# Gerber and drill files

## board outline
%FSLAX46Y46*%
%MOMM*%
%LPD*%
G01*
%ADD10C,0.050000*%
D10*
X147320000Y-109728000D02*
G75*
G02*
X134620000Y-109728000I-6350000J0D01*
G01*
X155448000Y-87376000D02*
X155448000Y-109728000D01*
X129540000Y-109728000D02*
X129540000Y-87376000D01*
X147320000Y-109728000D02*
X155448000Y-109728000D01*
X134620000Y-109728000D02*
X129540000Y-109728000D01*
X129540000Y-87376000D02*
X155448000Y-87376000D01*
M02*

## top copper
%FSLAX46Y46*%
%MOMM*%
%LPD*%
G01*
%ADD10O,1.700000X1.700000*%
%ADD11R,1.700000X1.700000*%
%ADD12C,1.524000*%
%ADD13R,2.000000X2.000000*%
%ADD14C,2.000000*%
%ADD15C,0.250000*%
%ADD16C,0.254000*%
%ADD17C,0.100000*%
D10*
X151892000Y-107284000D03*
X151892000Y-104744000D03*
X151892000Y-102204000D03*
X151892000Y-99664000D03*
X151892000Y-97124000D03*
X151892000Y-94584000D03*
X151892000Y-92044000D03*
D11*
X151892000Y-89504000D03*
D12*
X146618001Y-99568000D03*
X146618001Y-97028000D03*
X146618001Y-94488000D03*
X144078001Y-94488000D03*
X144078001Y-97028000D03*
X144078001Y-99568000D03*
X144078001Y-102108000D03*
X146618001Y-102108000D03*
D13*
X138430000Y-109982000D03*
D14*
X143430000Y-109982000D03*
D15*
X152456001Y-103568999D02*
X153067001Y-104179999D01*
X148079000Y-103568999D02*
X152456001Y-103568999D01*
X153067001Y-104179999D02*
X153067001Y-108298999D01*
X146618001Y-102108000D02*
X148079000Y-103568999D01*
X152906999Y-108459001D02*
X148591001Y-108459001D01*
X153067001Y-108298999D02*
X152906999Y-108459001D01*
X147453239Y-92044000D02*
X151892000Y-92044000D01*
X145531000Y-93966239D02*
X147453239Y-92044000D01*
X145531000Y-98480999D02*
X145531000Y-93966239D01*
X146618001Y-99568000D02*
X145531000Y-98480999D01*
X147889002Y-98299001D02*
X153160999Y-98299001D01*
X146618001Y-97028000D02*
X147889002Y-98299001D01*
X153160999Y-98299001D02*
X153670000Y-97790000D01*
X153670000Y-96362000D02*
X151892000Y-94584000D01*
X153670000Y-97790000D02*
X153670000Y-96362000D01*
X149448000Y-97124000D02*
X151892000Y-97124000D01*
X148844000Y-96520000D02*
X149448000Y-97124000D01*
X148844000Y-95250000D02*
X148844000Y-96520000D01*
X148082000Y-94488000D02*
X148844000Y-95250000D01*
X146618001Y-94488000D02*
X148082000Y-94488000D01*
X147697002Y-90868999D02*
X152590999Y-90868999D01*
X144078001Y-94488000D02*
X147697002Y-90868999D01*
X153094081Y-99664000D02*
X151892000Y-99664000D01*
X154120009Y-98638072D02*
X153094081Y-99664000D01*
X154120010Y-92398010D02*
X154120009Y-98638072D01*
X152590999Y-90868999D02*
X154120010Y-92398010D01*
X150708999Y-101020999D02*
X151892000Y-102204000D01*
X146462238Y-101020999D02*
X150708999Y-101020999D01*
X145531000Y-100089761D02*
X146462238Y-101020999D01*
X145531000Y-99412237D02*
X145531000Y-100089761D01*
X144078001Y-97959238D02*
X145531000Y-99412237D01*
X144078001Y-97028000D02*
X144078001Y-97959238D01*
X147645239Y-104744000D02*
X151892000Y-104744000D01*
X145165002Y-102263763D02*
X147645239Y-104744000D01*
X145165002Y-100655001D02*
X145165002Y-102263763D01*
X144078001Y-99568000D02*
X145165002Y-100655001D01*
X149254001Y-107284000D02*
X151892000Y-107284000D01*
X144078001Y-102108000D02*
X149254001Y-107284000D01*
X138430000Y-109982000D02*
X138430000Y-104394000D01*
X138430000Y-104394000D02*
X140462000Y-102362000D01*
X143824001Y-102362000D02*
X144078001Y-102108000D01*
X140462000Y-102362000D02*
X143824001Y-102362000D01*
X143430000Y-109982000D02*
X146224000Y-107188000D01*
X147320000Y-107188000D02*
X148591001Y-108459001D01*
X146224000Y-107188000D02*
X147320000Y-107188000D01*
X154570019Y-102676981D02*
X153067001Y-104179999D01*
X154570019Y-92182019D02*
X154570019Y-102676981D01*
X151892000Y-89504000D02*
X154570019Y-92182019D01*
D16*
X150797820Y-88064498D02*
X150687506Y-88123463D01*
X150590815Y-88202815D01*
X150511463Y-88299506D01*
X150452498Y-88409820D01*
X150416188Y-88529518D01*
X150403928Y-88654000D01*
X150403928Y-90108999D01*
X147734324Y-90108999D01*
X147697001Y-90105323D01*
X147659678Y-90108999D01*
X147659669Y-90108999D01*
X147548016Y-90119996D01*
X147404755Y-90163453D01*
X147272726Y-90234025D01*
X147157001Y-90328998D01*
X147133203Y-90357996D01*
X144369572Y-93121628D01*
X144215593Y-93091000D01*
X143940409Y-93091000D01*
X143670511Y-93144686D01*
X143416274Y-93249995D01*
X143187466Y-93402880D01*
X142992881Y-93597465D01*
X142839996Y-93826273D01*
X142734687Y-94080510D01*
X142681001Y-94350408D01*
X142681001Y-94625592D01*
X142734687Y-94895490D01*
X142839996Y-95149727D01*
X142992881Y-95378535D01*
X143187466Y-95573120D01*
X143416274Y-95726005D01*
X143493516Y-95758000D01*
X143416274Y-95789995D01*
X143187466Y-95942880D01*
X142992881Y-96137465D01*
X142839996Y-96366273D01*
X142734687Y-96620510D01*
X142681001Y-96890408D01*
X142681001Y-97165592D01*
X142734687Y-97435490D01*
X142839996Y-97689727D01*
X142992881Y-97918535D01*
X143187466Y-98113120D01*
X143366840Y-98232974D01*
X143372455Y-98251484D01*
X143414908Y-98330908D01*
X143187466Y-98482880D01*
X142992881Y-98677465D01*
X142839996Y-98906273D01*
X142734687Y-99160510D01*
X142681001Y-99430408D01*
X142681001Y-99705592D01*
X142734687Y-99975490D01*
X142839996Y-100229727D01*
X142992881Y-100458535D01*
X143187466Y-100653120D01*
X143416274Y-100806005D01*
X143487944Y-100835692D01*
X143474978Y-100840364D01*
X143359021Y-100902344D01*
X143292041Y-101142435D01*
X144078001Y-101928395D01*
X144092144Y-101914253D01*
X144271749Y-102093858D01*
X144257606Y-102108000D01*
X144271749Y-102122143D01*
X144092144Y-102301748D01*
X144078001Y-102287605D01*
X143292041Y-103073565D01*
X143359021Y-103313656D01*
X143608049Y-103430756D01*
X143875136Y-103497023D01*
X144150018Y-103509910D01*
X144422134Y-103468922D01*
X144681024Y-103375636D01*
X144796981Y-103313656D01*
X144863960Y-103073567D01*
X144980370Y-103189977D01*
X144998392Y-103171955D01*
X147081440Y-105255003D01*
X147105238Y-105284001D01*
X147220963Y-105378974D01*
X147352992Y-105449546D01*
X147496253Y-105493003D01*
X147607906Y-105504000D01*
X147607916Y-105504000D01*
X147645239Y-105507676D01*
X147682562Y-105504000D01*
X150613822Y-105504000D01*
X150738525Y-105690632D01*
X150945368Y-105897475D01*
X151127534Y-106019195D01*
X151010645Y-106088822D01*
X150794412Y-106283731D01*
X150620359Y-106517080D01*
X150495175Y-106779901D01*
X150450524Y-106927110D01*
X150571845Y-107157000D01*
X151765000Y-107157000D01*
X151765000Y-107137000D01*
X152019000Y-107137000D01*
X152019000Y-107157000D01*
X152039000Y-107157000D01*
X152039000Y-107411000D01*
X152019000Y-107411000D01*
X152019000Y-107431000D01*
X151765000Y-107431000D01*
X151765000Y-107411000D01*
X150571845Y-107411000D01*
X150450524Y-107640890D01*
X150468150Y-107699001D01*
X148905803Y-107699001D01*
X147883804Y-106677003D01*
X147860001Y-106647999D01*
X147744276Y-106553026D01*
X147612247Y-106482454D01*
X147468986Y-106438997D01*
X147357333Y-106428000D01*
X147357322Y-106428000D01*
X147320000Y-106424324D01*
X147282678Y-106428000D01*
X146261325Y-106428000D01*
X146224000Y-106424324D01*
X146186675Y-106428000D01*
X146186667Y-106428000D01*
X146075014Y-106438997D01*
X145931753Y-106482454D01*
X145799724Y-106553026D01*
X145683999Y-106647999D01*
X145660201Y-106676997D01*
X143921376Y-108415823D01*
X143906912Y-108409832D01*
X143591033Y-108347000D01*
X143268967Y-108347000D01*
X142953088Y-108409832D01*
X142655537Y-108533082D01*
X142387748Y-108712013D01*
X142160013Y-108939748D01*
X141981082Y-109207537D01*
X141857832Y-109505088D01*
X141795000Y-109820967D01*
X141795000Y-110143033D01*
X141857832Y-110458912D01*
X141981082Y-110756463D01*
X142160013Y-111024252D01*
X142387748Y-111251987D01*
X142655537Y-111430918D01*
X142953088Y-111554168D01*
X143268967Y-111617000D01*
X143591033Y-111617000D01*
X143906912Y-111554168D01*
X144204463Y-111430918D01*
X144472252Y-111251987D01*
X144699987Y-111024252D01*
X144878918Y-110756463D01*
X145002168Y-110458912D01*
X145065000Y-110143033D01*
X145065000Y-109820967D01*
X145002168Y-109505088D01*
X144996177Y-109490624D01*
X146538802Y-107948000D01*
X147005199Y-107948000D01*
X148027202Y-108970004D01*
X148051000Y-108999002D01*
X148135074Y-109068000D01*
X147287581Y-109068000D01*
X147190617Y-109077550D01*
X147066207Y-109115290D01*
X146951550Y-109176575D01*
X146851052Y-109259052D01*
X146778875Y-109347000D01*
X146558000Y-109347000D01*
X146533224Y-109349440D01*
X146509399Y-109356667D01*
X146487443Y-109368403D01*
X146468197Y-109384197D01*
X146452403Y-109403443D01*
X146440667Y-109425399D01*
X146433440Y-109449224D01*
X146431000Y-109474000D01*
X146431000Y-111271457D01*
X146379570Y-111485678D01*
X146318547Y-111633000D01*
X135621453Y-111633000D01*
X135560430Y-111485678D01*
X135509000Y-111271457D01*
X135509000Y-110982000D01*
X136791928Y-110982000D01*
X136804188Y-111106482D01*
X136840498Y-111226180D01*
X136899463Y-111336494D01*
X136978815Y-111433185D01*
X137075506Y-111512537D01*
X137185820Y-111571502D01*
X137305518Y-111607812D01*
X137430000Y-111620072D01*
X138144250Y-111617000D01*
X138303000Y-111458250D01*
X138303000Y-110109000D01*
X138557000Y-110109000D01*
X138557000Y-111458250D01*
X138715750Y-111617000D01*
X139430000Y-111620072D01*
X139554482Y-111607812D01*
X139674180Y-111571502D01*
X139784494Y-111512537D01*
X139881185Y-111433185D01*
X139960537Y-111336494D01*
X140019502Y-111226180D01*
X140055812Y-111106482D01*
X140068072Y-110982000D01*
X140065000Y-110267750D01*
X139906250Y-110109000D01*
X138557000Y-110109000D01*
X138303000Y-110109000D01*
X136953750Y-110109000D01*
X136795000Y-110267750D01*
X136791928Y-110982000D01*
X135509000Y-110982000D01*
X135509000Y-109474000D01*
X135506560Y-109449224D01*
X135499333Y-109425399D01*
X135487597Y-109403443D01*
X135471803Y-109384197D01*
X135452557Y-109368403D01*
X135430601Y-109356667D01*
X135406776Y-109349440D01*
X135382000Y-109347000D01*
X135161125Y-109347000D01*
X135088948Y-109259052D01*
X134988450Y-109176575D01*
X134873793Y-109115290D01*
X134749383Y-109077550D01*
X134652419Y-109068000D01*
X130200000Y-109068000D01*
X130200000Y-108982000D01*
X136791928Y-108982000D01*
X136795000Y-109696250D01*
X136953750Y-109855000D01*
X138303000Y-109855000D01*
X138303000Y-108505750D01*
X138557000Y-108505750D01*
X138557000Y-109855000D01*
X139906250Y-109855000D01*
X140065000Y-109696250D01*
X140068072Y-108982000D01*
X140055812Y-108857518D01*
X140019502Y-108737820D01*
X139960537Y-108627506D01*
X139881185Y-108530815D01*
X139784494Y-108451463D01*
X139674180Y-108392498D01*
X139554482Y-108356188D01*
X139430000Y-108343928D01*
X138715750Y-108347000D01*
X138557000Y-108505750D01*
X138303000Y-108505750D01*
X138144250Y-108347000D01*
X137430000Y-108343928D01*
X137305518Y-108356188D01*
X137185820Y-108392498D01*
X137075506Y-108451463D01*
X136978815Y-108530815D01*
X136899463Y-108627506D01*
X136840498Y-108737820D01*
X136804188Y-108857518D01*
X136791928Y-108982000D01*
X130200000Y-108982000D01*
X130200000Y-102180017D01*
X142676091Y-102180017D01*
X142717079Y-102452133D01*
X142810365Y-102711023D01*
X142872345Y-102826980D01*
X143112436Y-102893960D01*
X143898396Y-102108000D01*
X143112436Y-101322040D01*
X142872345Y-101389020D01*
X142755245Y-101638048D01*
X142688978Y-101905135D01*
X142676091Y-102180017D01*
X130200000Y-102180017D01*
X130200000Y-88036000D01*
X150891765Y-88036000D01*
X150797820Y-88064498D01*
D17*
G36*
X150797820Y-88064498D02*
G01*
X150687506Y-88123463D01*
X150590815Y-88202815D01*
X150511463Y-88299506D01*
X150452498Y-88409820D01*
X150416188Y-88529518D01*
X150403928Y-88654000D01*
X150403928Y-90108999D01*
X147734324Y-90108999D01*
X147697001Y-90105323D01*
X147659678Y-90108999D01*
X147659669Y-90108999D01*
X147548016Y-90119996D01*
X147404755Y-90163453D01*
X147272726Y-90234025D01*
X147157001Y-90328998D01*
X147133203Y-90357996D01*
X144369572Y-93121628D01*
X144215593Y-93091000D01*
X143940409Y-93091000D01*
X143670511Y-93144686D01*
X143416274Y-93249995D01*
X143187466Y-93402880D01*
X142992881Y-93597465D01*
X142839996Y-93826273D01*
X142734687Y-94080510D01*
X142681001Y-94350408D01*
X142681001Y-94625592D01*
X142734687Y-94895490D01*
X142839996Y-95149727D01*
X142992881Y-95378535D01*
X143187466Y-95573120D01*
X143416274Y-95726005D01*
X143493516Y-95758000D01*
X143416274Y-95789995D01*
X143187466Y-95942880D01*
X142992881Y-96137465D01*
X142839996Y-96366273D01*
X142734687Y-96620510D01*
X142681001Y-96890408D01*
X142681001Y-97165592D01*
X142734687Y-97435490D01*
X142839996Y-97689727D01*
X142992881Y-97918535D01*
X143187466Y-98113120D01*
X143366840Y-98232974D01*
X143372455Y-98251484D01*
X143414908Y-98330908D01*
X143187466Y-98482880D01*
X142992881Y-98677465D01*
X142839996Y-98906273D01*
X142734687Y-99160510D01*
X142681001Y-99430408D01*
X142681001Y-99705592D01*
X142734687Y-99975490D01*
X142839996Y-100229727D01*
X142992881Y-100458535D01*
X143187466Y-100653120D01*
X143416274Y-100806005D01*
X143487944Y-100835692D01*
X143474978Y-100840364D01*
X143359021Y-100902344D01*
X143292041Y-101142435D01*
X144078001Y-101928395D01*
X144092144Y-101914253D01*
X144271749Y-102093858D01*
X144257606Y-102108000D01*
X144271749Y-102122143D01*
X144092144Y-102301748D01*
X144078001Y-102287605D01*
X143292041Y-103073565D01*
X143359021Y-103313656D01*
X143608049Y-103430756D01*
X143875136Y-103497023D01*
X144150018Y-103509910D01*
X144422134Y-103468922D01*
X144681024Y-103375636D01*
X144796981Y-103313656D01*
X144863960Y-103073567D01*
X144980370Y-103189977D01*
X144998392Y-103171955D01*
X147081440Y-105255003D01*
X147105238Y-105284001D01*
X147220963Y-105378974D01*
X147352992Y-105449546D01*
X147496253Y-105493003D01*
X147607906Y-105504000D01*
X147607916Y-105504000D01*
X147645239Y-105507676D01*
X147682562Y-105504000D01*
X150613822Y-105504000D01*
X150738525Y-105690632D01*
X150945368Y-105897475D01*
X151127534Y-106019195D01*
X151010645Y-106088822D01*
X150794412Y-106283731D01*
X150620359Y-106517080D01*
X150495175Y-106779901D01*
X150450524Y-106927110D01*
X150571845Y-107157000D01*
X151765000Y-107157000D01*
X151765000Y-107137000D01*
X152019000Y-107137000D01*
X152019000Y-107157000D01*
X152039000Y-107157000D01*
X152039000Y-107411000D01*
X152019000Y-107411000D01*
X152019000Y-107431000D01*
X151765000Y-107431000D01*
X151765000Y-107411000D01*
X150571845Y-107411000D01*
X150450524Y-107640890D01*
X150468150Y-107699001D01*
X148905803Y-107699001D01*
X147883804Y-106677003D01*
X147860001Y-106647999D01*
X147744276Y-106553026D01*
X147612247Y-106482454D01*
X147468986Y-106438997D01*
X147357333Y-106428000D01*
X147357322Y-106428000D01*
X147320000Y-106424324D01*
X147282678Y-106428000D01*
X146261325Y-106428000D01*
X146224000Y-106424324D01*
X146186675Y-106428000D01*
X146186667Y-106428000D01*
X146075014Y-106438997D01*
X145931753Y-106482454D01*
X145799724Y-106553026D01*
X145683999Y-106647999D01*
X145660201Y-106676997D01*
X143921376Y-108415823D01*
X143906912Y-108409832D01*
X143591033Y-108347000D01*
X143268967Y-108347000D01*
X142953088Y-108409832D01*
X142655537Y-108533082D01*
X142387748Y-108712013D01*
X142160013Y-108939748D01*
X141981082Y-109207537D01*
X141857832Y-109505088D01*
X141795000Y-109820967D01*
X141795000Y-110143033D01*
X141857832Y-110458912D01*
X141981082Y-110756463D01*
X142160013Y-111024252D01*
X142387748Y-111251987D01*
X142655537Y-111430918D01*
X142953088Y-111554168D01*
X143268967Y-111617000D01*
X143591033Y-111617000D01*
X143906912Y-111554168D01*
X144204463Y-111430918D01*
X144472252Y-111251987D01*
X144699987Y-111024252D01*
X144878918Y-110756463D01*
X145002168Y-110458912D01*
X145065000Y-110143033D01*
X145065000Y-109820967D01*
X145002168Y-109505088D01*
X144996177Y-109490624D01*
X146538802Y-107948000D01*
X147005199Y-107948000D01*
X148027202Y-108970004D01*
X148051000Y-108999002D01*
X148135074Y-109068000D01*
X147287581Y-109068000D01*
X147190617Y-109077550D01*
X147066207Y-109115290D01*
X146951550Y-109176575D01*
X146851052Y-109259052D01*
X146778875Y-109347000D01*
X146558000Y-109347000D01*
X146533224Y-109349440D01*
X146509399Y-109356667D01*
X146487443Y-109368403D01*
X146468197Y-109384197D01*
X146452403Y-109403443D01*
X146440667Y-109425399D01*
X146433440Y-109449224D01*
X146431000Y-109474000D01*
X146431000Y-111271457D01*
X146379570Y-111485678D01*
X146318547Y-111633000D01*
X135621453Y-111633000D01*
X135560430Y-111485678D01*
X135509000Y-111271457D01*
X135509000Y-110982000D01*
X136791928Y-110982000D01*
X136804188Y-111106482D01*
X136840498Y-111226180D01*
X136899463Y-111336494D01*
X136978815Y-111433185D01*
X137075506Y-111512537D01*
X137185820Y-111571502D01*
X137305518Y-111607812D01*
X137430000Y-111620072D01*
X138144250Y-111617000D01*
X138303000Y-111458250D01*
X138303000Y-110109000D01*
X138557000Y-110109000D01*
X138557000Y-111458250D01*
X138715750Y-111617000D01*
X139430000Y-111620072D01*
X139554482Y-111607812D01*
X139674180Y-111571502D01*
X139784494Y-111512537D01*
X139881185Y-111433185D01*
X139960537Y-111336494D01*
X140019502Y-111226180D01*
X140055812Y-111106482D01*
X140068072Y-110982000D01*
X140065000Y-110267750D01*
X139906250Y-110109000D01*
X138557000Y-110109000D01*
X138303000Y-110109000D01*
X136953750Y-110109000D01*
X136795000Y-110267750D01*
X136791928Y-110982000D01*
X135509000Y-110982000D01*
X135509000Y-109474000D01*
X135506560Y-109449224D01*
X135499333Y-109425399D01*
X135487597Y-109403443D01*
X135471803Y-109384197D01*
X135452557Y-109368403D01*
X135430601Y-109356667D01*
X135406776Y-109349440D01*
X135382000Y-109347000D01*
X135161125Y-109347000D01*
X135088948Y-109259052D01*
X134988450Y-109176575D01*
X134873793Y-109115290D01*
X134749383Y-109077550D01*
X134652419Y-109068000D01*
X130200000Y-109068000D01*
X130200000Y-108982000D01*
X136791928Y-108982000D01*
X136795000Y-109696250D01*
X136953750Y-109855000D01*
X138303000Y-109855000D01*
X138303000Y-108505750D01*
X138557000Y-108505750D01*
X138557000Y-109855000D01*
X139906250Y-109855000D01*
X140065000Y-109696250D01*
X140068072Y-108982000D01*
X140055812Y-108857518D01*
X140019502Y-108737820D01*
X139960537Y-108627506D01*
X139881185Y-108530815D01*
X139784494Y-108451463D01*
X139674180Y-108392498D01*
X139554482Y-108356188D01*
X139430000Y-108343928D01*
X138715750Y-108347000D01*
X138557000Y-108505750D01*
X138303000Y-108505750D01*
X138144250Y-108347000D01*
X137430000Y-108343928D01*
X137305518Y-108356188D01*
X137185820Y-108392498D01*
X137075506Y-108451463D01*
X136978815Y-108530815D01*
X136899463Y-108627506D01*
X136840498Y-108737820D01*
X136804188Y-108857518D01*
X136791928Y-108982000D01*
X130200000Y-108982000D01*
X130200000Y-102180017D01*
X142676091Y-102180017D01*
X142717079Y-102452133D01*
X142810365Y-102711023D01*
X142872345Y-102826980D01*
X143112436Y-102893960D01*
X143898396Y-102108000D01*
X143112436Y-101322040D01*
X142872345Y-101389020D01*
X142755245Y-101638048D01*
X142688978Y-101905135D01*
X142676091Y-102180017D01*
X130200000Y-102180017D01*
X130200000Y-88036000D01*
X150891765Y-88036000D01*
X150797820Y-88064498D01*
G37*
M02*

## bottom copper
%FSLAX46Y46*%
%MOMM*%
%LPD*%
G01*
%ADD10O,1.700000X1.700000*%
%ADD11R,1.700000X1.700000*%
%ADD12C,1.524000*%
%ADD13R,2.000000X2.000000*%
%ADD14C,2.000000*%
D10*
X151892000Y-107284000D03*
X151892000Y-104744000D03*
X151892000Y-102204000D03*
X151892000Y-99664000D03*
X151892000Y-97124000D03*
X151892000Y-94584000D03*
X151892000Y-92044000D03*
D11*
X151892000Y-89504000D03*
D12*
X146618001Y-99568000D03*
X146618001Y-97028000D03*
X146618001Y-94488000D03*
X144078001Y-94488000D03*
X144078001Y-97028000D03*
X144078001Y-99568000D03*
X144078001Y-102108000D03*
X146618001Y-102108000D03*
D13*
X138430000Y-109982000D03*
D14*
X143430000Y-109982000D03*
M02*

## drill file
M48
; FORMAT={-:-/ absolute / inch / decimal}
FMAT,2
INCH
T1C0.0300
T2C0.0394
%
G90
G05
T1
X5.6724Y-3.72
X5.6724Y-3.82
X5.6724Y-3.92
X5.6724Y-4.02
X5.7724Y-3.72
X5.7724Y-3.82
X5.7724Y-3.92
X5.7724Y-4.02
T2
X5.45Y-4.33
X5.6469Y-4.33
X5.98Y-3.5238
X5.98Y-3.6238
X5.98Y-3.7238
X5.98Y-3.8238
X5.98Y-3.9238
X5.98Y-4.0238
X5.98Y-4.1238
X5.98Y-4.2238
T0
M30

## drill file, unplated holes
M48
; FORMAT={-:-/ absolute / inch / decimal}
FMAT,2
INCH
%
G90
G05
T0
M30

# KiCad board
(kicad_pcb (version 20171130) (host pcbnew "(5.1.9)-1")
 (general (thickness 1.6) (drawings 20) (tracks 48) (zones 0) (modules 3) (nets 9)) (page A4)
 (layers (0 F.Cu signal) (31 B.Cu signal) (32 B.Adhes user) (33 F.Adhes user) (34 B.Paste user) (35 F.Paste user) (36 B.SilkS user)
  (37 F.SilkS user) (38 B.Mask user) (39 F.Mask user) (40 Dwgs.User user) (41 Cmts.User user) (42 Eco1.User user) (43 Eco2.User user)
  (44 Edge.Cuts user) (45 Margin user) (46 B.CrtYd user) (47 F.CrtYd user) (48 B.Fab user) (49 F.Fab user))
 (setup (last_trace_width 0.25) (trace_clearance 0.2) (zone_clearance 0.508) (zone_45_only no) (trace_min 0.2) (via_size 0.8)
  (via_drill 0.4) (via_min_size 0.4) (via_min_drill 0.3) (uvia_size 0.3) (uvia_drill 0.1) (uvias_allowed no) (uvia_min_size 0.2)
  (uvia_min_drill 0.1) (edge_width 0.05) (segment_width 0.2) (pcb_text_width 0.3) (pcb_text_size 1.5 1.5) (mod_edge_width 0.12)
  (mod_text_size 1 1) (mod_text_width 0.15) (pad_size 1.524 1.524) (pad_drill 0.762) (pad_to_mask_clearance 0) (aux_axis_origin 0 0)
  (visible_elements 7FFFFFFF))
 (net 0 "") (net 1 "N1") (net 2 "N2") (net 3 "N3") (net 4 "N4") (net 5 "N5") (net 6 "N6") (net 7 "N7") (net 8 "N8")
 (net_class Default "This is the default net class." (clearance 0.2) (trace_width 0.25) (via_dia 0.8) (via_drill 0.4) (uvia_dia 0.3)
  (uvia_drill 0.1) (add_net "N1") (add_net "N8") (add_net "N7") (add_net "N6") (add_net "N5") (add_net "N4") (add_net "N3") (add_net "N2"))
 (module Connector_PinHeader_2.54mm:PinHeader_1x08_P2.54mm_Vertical (layer F.Cu) (at 151.892 89.504)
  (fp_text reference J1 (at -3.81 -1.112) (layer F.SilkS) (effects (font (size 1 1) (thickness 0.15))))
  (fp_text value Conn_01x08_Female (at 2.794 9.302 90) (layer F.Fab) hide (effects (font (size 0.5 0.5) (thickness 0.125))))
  (pad 8 thru_hole oval (at 0 17.78) (size 1.7 1.7) (drill 1) (layers *.Cu *.Mask) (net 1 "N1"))
  (pad 7 thru_hole oval (at 0 15.24) (size 1.7 1.7) (drill 1) (layers *.Cu *.Mask) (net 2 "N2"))
  (pad 6 thru_hole oval (at 0 12.7) (size 1.7 1.7) (drill 1) (layers *.Cu *.Mask) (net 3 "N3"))
  (pad 5 thru_hole oval (at 0 10.16) (size 1.7 1.7) (drill 1) (layers *.Cu *.Mask) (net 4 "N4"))
  (pad 4 thru_hole oval (at 0 7.62) (size 1.7 1.7) (drill 1) (layers *.Cu *.Mask) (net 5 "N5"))
  (pad 3 thru_hole oval (at 0 5.08) (size 1.7 1.7) (drill 1) (layers *.Cu *.Mask) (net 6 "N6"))
  (pad 2 thru_hole oval (at 0 2.54) (size 1.7 1.7) (drill 1) (layers *.Cu *.Mask) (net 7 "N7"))
  (pad 1 thru_hole rect (at 0 0) (size 1.7 1.7) (drill 1) (layers *.Cu *.Mask) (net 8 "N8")))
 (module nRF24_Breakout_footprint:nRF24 (layer F.Cu) (at 138.998001 99.568)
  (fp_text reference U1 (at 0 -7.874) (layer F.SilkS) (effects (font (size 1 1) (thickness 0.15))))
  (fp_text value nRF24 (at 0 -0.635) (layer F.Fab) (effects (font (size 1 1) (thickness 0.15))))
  (pad 1 thru_hole circle (at 7.62 0) (size 1.524 1.524) (drill 0.762) (layers *.Cu *.Mask) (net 7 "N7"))
  (pad 2 thru_hole circle (at 7.62 -2.54) (size 1.524 1.524) (drill 0.762) (layers *.Cu *.Mask) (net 6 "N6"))
  (pad 3 thru_hole circle (at 7.62 -5.08) (size 1.524 1.524) (drill 0.762) (layers *.Cu *.Mask) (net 5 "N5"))
  (pad 4 thru_hole circle (at 5.08 -5.08) (size 1.524 1.524) (drill 0.762) (layers *.Cu *.Mask) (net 4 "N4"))
  (pad 5 thru_hole circle (at 5.08 -2.54) (size 1.524 1.524) (drill 0.762) (layers *.Cu *.Mask) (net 3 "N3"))
  (pad 6 thru_hole circle (at 5.08 0) (size 1.524 1.524) (drill 0.762) (layers *.Cu *.Mask) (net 2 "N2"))
  (pad 7 thru_hole circle (at 5.08 2.54) (size 1.524 1.524) (drill 0.762) (layers *.Cu *.Mask) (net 1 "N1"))
  (pad 0 thru_hole circle (at 7.62 2.54) (size 1.524 1.524) (drill 0.762) (layers *.Cu *.Mask) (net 8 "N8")))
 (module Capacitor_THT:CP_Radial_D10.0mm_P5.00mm (layer F.Cu) (at 138.43 109.982)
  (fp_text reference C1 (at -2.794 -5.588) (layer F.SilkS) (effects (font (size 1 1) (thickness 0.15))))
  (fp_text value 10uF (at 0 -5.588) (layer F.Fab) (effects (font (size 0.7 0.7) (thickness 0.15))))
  (pad 1 thru_hole rect (at 0 0) (size 2 2) (drill 1) (layers *.Cu *.Mask) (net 1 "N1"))
  (pad 2 thru_hole circle (at 5 0) (size 2 2) (drill 1) (layers *.Cu *.Mask) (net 8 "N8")))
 (gr_arc (start 140.97 109.728) (end 134.62 109.728) (angle -180) (layer Edge.Cuts) (width 0.05))
 (gr_line (start 155.448 87.376) (end 155.448 109.728) (layer Edge.Cuts) (width 0.05))
 (gr_line (start 129.54 109.728) (end 129.54 87.376) (layer Edge.Cuts) (width 0.05))
 (gr_line (start 147.32 109.728) (end 155.448 109.728) (layer Edge.Cuts) (width 0.05))
 (gr_line (start 134.62 109.728) (end 129.54 109.728) (layer Edge.Cuts) (width 0.05))
 (gr_line (start 129.54 87.376) (end 155.448 87.376) (layer Edge.Cuts) (width 0.05))
 (segment (start 152.456001 103.568999) (end 153.067001 104.179999) (width 0.25) (layer F.Cu) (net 8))
 (segment (start 148.079 103.568999) (end 152.456001 103.568999) (width 0.25) (layer F.Cu) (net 8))
 (segment (start 153.067001 104.179999) (end 153.067001 108.298999) (width 0.25) (layer F.Cu) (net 8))
 (segment (start 146.618001 102.108) (end 148.079 103.568999) (width 0.25) (layer F.Cu) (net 8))
 (segment (start 152.906999 108.459001) (end 148.591001 108.459001) (width 0.25) (layer F.Cu) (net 8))
 (segment (start 153.067001 108.298999) (end 152.906999 108.459001) (width 0.25) (layer F.Cu) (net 8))
 (segment (start 147.453239 92.044) (end 151.892 92.044) (width 0.25) (layer F.Cu) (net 7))
 (segment (start 145.531 93.966239) (end 147.453239 92.044) (width 0.25) (layer F.Cu) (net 7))
 (segment (start 145.531 98.480999) (end 145.531 93.966239) (width 0.25) (layer F.Cu) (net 7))
 (segment (start 146.618001 99.568) (end 145.531 98.480999) (width 0.25) (layer F.Cu) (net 7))
 (segment (start 147.889002 98.299001) (end 153.160999 98.299001) (width 0.25) (layer F.Cu) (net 6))
 (segment (start 146.618001 97.028) (end 147.889002 98.299001) (width 0.25) (layer F.Cu) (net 6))
 (segment (start 153.160999 98.299001) (end 153.67 97.79) (width 0.25) (layer F.Cu) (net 6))
 (segment (start 153.67 96.362) (end 151.892 94.584) (width 0.25) (layer F.Cu) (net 6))
 (segment (start 153.67 97.79) (end 153.67 96.362) (width 0.25) (layer F.Cu) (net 6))
 (segment (start 149.448 97.124) (end 151.892 97.124) (width 0.25) (layer F.Cu) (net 5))
 (segment (start 148.844 96.52) (end 149.448 97.124) (width 0.25) (layer F.Cu) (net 5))
 (segment (start 148.844 95.25) (end 148.844 96.52) (width 0.25) (layer F.Cu) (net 5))
 (segment (start 148.082 94.488) (end 148.844 95.25) (width 0.25) (layer F.Cu) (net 5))
 (segment (start 146.618001 94.488) (end 148.082 94.488) (width 0.25) (layer F.Cu) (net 5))
 (segment (start 147.697002 90.868999) (end 152.590999 90.868999) (width 0.25) (layer F.Cu) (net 4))
 (segment (start 144.078001 94.488) (end 147.697002 90.868999) (width 0.25) (layer F.Cu) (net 4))
 (segment (start 153.094081 99.664) (end 151.892 99.664) (width 0.25) (layer F.Cu) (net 4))
 (segment (start 154.120009 98.638072) (end 153.094081 99.664) (width 0.25) (layer F.Cu) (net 4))
 (segment (start 154.12001 92.39801) (end 154.120009 98.638072) (width 0.25) (layer F.Cu) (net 4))
 (segment (start 152.590999 90.868999) (end 154.12001 92.39801) (width 0.25) (layer F.Cu) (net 4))
 (segment (start 150.708999 101.020999) (end 151.892 102.204) (width 0.25) (layer F.Cu) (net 3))
 (segment (start 146.462238 101.020999) (end 150.708999 101.020999) (width 0.25) (layer F.Cu) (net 3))
 (segment (start 145.531 100.089761) (end 146.462238 101.020999) (width 0.25) (layer F.Cu) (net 3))
 (segment (start 145.531 99.412237) (end 145.531 100.089761) (width 0.25) (layer F.Cu) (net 3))
 (segment (start 144.078001 97.959238) (end 145.531 99.412237) (width 0.25) (layer F.Cu) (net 3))
 (segment (start 144.078001 97.028) (end 144.078001 97.959238) (width 0.25) (layer F.Cu) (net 3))
 (segment (start 147.645239 104.744) (end 151.892 104.744) (width 0.25) (layer F.Cu) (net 2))
 (segment (start 145.165002 102.263763) (end 147.645239 104.744) (width 0.25) (layer F.Cu) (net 2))
 (segment (start 145.165002 100.655001) (end 145.165002 102.263763) (width 0.25) (layer F.Cu) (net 2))
 (segment (start 144.078001 99.568) (end 145.165002 100.655001) (width 0.25) (layer F.Cu) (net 2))
 (segment (start 149.254001 107.284) (end 151.892 107.284) (width 0.25) (layer F.Cu) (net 1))
 (segment (start 144.078001 102.108) (end 149.254001 107.284) (width 0.25) (layer F.Cu) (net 1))
 (segment (start 138.43 109.982) (end 138.43 104.394) (width 0.25) (layer F.Cu) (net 1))
 (segment (start 138.43 104.394) (end 140.462 102.362) (width 0.25) (layer F.Cu) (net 1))
 (segment (start 143.824001 102.362) (end 144.078001 102.108) (width 0.25) (layer F.Cu) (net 1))
 (segment (start 140.462 102.362) (end 143.824001 102.362) (width 0.25) (layer F.Cu) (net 1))
 (segment (start 143.43 109.982) (end 146.224 107.188) (width 0.25) (layer F.Cu) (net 8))
 (segment (start 147.32 107.188) (end 148.591001 108.459001) (width 0.25) (layer F.Cu) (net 8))
 (segment (start 146.224 107.188) (end 147.32 107.188) (width 0.25) (layer F.Cu) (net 8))
 (segment (start 154.570019 102.676981) (end 153.067001 104.179999) (width 0.25) (layer F.Cu) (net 8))
 (segment (start 154.570019 92.182019) (end 154.570019 102.676981) (width 0.25) (layer F.Cu) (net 8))
 (segment (start 151.892 89.504) (end 154.570019 92.182019) (width 0.25) (layer F.Cu) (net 8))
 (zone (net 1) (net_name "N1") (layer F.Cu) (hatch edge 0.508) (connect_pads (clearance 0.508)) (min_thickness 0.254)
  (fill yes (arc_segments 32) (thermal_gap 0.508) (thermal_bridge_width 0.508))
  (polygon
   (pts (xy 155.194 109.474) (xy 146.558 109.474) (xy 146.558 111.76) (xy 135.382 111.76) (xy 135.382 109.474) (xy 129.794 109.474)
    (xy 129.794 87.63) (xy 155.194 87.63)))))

